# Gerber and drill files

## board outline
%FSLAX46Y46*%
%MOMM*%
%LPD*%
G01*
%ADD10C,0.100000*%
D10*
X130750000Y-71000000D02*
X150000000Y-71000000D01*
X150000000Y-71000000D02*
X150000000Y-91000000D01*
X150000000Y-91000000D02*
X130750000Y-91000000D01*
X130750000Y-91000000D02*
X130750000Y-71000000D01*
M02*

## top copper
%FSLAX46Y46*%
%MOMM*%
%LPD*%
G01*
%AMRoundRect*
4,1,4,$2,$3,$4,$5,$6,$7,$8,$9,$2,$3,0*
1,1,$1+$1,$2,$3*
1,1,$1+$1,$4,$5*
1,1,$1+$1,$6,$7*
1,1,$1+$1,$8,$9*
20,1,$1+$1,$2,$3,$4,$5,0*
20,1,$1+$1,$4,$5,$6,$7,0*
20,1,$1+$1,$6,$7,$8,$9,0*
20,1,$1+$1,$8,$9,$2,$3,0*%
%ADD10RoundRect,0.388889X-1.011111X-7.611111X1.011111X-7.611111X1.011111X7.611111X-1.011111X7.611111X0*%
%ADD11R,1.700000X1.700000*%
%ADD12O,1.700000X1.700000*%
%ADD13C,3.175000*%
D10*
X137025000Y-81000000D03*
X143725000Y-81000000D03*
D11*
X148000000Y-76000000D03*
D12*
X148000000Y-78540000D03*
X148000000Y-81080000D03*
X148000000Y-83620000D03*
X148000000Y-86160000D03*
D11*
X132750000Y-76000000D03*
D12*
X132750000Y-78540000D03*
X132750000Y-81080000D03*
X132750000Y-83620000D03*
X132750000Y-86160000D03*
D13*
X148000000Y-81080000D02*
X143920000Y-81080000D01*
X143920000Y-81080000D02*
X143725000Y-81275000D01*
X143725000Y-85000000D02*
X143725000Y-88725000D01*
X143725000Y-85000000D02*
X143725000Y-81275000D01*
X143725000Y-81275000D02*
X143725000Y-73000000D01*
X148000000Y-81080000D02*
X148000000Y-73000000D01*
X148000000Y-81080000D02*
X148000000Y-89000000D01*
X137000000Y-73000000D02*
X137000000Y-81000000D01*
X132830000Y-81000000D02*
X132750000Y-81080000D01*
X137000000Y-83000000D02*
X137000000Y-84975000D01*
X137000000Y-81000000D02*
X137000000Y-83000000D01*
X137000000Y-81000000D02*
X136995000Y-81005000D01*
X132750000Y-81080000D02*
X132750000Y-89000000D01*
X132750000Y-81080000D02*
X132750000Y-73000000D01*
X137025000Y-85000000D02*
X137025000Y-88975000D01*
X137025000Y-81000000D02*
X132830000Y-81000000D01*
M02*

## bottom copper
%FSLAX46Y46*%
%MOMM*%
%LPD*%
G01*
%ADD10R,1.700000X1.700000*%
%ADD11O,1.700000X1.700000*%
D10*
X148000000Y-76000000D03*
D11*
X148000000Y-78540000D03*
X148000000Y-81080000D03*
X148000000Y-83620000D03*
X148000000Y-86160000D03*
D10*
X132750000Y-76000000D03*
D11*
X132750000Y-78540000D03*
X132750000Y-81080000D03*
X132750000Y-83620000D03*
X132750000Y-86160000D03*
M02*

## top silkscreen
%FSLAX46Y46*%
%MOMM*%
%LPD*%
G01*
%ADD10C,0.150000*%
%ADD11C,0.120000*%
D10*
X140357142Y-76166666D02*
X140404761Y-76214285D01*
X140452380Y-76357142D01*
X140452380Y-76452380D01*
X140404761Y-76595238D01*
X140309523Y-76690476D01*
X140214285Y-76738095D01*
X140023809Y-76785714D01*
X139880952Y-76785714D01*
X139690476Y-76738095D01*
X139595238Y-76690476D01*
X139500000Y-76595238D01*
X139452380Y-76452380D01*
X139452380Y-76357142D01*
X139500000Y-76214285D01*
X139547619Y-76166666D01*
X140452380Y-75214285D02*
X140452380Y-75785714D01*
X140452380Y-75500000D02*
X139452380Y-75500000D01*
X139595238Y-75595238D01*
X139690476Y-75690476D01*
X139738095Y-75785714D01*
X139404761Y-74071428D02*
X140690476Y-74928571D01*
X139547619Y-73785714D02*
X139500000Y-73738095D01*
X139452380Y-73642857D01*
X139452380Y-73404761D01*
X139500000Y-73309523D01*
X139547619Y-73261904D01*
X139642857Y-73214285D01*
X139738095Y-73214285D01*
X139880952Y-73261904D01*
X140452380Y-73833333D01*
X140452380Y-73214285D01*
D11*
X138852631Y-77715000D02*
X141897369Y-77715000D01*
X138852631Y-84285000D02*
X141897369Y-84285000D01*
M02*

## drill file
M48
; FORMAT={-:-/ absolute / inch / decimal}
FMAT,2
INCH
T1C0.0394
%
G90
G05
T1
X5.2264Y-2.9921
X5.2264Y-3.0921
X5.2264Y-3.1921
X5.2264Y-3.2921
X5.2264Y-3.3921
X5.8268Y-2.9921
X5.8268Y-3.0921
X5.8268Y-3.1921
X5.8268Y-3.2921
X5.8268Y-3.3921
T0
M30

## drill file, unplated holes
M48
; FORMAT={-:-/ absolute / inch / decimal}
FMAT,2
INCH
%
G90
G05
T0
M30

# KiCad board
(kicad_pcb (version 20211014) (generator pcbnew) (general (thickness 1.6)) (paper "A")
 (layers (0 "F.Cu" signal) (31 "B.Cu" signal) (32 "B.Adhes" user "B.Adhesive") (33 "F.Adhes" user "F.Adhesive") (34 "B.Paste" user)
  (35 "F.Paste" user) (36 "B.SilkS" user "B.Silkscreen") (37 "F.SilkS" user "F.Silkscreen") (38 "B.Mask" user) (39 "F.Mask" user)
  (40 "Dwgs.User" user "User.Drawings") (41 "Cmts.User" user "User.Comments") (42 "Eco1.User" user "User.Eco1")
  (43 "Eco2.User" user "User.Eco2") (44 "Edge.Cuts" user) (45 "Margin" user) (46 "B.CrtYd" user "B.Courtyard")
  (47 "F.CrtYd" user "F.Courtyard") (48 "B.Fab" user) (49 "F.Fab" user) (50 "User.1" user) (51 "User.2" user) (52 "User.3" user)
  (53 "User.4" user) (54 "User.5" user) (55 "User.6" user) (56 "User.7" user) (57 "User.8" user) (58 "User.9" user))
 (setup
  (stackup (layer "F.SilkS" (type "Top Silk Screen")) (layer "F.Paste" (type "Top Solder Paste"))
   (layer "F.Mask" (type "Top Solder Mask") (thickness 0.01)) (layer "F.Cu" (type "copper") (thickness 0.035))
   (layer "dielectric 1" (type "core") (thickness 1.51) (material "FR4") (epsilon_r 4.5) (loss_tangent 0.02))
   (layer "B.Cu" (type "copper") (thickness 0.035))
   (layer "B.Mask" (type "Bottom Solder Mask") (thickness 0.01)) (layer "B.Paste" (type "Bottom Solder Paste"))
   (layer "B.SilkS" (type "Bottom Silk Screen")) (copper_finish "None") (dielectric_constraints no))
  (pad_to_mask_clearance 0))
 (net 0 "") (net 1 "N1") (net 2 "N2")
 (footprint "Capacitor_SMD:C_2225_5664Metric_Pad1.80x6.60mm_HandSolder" (layer "F.Cu") (at 140.375 81)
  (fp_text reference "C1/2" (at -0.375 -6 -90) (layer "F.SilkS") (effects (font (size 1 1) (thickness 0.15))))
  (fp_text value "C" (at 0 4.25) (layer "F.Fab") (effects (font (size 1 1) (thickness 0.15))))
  (fp_line (start -1.522369 -3.285) (end 1.522369 -3.285) (layer "F.SilkS") (width 0.12))
  (fp_line (start -1.522369 3.285) (end 1.522369 3.285) (layer "F.SilkS") (width 0.12))
  (pad "1" smd roundrect (at -3.35 0) (size 2.8 16) (layers "F.Cu" "F.Paste" "F.Mask") (roundrect_rratio 0.138889) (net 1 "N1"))
  (pad "2" smd roundrect (at 3.35 0) (size 2.8 16) (layers "F.Cu" "F.Paste" "F.Mask") (roundrect_rratio 0.138889) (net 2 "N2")))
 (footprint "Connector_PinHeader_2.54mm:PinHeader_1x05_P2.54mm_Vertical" (layer "B.Cu") (at 148 76 180)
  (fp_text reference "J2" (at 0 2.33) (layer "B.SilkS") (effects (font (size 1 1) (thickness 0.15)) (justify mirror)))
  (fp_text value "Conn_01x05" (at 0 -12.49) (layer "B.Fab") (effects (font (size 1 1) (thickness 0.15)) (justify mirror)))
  (pad "1" thru_hole rect (at 0 0 180) (size 1.7 1.7) (drill 1) (layers *.Cu *.Mask) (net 2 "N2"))
  (pad "2" thru_hole oval (at 0 -2.54 180) (size 1.7 1.7) (drill 1) (layers *.Cu *.Mask) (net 2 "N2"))
  (pad "3" thru_hole oval (at 0 -5.08 180) (size 1.7 1.7) (drill 1) (layers *.Cu *.Mask) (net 2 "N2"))
  (pad "4" thru_hole oval (at 0 -7.62 180) (size 1.7 1.7) (drill 1) (layers *.Cu *.Mask) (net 2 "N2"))
  (pad "5" thru_hole oval (at 0 -10.16 180) (size 1.7 1.7) (drill 1) (layers *.Cu *.Mask) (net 2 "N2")))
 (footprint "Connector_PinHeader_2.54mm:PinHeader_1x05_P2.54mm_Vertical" (layer "B.Cu") (at 132.75 76 180)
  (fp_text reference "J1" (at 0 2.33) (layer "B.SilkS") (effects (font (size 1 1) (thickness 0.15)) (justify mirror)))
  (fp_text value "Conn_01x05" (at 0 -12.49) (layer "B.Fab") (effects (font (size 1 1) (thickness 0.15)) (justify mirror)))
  (pad "1" thru_hole rect (at 0 0 180) (size 1.7 1.7) (drill 1) (layers *.Cu *.Mask) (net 1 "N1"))
  (pad "2" thru_hole oval (at 0 -2.54 180) (size 1.7 1.7) (drill 1) (layers *.Cu *.Mask) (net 1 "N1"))
  (pad "3" thru_hole oval (at 0 -5.08 180) (size 1.7 1.7) (drill 1) (layers *.Cu *.Mask) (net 1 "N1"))
  (pad "4" thru_hole oval (at 0 -7.62 180) (size 1.7 1.7) (drill 1) (layers *.Cu *.Mask) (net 1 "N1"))
  (pad "5" thru_hole oval (at 0 -10.16 180) (size 1.7 1.7) (drill 1) (layers *.Cu *.Mask) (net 1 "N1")))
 (gr_rect (start 130.75 71) (end 150 91) (layer "Edge.Cuts") (width 0.1) (fill none))
 (segment (start 148 81.08) (end 143.92 81.08) (width 3.175) (layer "F.Cu") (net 2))
 (segment (start 143.92 81.08) (end 143.725 81.275) (width 3.175) (layer "F.Cu") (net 2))
 (segment (start 143.725 85) (end 143.725 88.725) (width 3.175) (layer "F.Cu") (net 2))
 (segment (start 143.725 85) (end 143.725 81.275) (width 3.175) (layer "F.Cu") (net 2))
 (segment (start 143.725 81.275) (end 143.725 73) (width 3.175) (layer "F.Cu") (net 2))
 (segment (start 148 81.08) (end 148 73) (width 3.175) (layer "F.Cu") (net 2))
 (segment (start 148 81.08) (end 148 89) (width 3.175) (layer "F.Cu") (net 2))
 (segment (start 137 73) (end 137 81) (width 3.175) (layer "F.Cu") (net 1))
 (segment (start 132.83 81) (end 132.75 81.08) (width 3.175) (layer "F.Cu") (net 1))
 (segment (start 137 83) (end 137 84.975) (width 3.175) (layer "F.Cu") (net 1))
 (segment (start 137 81) (end 137 83) (width 3.175) (layer "F.Cu") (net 1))
 (segment (start 137 81) (end 136.995 81.005) (width 3.175) (layer "F.Cu") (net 1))
 (segment (start 132.75 81.08) (end 132.75 89) (width 3.175) (layer "F.Cu") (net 1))
 (segment (start 132.75 81.08) (end 132.75 73) (width 3.175) (layer "F.Cu") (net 1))
 (segment (start 137.025 85) (end 137.025 88.975) (width 3.175) (layer "F.Cu") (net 1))
 (segment (start 137.025 81) (end 132.83 81) (width 3.175) (layer "F.Cu") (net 1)))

